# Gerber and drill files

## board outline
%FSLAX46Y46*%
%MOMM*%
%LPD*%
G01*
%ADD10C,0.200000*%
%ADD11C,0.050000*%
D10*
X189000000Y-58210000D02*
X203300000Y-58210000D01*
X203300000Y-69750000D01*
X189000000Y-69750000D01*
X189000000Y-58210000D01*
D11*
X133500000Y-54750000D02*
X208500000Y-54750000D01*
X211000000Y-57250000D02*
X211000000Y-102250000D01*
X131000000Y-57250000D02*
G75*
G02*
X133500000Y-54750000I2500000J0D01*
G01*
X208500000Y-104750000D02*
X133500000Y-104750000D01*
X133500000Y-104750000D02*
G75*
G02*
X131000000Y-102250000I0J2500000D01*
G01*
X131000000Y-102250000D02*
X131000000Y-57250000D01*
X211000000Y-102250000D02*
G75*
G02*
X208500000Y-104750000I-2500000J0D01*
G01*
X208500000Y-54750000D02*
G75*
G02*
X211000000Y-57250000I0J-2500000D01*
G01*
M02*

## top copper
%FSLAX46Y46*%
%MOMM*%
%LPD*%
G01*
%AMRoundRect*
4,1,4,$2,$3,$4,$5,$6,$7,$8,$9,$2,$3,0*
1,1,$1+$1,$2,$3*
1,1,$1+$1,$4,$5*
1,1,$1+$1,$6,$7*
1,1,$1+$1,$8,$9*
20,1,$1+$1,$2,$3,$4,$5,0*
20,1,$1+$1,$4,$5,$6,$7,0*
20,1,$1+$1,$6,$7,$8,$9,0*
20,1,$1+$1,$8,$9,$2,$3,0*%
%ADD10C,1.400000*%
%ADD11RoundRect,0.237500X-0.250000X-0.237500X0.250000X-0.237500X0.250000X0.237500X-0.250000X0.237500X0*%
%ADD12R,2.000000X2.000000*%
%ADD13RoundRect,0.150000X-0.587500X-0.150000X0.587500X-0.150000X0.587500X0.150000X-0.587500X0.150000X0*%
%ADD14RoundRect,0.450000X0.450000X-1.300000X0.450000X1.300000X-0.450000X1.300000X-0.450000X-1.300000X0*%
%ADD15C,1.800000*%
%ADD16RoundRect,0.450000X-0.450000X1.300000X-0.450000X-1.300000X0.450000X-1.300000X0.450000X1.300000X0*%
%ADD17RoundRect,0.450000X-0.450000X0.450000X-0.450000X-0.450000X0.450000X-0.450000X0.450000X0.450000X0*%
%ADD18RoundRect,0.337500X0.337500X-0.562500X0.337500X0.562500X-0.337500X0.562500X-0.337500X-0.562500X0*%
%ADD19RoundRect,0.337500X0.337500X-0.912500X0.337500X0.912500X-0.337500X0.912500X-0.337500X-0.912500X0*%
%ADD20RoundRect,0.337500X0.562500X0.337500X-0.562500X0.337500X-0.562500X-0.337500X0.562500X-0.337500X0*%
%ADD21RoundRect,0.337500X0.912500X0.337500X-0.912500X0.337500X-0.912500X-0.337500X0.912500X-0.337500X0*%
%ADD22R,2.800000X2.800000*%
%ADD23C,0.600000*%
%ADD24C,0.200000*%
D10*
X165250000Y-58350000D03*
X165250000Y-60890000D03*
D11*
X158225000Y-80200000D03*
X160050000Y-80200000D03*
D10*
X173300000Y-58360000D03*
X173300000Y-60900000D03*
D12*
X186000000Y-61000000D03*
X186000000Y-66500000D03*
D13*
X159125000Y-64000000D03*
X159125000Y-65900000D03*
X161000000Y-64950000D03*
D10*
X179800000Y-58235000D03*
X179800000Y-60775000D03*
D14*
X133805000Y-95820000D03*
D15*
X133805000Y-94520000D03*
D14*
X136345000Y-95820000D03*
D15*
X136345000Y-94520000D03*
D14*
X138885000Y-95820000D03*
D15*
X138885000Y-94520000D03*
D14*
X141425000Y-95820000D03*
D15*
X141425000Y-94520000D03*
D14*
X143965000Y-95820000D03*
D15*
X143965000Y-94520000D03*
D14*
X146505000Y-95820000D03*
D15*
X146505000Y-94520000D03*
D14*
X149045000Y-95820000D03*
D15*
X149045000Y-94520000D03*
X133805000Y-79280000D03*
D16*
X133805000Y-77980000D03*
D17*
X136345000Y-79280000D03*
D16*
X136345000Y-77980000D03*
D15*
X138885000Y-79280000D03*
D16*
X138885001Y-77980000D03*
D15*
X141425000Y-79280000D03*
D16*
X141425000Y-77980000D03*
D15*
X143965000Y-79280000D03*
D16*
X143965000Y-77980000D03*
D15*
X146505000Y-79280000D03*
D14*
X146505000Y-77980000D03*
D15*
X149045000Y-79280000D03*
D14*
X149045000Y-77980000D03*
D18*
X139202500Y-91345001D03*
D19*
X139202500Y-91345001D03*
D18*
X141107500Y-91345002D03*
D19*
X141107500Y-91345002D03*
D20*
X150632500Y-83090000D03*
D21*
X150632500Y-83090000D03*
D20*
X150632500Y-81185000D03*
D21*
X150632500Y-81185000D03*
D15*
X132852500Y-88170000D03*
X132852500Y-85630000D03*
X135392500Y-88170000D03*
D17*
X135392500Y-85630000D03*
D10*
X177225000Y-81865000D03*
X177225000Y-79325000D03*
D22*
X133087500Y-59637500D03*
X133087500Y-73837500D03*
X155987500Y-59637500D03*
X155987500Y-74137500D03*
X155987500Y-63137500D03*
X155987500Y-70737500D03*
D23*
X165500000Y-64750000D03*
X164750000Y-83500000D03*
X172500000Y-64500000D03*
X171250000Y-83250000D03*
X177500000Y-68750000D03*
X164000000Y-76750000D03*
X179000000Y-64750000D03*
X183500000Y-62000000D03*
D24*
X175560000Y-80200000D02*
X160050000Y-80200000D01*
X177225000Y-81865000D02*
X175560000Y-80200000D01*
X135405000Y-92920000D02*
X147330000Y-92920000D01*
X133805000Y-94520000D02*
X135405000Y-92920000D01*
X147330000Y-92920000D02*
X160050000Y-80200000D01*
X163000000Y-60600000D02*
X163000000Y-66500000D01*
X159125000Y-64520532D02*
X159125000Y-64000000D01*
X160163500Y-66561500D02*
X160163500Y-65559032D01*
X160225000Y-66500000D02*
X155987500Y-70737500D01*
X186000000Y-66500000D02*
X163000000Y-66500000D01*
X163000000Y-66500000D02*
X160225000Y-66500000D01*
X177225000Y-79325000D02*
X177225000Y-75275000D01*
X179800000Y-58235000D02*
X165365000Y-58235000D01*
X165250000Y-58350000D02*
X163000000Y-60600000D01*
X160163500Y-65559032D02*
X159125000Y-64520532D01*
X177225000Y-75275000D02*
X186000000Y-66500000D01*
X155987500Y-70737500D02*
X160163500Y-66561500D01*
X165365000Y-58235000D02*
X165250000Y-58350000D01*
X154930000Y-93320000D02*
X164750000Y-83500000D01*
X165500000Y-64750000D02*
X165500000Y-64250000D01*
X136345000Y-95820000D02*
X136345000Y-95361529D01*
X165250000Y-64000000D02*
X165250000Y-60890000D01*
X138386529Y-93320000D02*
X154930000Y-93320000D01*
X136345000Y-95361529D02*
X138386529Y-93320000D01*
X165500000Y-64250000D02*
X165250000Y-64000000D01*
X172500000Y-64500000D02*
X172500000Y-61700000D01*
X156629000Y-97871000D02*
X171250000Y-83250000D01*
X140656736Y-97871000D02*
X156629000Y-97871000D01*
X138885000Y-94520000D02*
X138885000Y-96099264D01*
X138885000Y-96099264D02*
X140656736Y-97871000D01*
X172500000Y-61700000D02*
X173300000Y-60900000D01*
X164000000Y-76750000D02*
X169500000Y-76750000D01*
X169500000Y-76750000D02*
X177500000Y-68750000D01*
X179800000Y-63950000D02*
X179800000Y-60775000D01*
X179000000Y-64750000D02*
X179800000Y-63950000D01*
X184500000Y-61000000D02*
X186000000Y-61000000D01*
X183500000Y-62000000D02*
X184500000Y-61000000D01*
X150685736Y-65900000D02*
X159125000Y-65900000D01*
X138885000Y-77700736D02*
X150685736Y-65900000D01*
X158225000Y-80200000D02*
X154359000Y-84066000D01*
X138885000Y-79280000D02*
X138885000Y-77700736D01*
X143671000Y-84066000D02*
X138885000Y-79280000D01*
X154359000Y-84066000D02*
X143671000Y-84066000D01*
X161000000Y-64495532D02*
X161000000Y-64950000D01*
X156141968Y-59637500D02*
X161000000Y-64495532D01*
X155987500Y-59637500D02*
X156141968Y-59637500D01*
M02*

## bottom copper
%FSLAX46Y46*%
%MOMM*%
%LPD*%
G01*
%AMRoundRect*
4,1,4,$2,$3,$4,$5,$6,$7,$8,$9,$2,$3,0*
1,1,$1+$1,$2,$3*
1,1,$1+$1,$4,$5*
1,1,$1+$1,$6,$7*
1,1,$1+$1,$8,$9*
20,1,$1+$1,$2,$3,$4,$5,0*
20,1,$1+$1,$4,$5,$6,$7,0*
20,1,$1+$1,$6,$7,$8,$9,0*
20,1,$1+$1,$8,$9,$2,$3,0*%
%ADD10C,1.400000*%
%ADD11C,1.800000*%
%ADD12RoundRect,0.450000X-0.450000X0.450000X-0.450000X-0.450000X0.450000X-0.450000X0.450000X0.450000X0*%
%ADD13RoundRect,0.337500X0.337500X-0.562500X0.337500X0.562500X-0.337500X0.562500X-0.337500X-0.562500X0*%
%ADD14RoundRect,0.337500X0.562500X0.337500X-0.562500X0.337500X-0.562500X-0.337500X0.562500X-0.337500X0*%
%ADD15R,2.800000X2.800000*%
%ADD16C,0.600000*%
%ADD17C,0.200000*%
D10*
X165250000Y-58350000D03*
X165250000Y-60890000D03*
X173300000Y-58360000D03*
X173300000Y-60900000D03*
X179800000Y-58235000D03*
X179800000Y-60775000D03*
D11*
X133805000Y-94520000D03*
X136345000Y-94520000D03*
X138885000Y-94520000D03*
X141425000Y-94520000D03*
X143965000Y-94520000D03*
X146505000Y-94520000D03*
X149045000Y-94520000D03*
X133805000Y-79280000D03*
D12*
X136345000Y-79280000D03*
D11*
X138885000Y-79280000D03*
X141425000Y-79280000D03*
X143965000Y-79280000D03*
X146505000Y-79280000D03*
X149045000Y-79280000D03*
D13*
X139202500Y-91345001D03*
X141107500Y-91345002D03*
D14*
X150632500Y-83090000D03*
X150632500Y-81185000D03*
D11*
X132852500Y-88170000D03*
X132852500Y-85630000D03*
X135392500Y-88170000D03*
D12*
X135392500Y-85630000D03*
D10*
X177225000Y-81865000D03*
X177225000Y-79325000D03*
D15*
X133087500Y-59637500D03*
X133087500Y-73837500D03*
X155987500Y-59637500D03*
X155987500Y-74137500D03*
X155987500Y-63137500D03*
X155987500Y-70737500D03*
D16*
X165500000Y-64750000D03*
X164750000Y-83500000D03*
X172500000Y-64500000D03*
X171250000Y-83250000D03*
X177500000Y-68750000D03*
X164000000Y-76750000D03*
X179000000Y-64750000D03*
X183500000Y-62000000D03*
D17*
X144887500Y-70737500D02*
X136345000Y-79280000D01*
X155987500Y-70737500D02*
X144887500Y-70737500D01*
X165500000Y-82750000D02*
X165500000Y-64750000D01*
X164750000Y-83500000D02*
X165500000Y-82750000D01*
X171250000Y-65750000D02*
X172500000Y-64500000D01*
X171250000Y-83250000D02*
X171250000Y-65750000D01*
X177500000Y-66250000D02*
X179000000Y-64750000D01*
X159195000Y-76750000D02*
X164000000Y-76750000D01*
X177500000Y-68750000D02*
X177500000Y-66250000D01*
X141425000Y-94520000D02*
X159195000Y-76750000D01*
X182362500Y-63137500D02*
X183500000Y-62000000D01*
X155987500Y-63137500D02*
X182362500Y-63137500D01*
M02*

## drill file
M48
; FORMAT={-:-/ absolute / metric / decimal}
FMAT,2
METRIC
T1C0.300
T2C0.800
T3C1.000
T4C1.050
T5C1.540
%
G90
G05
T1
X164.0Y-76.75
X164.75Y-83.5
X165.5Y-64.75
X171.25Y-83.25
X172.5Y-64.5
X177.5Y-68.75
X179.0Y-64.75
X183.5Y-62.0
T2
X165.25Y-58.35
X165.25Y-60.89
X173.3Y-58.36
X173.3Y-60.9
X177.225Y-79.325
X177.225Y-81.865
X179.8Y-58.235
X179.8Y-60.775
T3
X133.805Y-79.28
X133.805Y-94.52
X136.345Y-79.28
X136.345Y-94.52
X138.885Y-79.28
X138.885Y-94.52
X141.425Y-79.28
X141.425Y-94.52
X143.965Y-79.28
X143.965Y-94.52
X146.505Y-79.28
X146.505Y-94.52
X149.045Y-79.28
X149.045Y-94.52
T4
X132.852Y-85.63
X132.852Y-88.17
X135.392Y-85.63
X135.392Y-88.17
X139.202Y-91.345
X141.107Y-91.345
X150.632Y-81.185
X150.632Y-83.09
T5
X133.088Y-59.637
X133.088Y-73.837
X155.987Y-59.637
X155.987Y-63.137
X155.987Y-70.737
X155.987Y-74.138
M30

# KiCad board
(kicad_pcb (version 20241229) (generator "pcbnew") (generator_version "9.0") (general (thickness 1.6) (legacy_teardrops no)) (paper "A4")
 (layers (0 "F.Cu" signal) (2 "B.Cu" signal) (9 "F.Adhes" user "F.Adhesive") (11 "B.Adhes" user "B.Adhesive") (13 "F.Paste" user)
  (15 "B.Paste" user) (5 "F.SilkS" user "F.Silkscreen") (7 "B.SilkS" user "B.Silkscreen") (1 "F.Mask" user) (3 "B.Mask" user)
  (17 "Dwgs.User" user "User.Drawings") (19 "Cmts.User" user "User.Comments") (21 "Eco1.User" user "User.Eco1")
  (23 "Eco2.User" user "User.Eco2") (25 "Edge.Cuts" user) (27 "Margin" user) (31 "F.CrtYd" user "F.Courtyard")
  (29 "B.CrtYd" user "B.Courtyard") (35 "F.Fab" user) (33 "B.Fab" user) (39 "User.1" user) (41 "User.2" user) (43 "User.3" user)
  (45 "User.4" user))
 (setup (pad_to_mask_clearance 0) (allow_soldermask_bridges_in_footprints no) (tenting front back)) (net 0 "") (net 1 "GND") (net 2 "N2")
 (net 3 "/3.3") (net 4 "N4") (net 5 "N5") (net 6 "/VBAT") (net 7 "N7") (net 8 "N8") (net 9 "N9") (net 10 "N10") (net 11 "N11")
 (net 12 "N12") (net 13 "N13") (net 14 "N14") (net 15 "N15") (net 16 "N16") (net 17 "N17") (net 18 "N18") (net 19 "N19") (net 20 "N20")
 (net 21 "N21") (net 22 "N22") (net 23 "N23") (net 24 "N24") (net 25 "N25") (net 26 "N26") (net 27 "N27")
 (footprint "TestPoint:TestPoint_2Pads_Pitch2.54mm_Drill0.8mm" (layer "F.Cu") (at 165.25 58.35 -90)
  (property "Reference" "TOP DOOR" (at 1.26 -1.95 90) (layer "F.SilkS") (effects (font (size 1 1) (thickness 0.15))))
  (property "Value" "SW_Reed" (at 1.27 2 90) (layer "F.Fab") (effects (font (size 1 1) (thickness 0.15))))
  (pad "1" thru_hole circle (at 0 0 270) (size 1.4 1.4) (drill 0.8) (layers "*.Cu" "*.Mask") (remove_unused_layers no) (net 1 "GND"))
  (pad "2" thru_hole circle (at 2.54 0 270) (size 1.4 1.4) (drill 0.8) (layers "*.Cu" "*.Mask") (remove_unused_layers no) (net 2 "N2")))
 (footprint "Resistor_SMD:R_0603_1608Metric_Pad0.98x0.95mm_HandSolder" (layer "F.Cu") (at 159.1375 80.2)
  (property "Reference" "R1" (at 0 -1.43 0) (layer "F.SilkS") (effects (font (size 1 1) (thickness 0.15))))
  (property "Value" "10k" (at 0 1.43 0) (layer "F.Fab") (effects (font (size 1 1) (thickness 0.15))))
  (pad "1" smd roundrect (at -0.9125 0) (size 0.975 0.95) (layers "F.Cu" "F.Mask" "F.Paste") (roundrect_rratio 0.25) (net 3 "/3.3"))
  (pad "2" smd roundrect (at 0.9125 0) (size 0.975 0.95) (layers "F.Cu" "F.Mask" "F.Paste") (roundrect_rratio 0.25) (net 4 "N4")))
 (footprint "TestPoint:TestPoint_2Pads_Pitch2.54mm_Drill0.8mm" (layer "F.Cu") (at 173.3 58.36 -90)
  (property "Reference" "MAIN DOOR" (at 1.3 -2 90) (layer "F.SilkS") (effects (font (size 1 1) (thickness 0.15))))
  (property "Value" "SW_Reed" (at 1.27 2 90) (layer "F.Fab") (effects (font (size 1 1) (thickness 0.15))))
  (pad "1" thru_hole circle (at 0 0 270) (size 1.4 1.4) (drill 0.8) (layers "*.Cu" "*.Mask") (remove_unused_layers no) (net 1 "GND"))
  (pad "2" thru_hole circle (at 2.54 0 270) (size 1.4 1.4) (drill 0.8) (layers "*.Cu" "*.Mask") (remove_unused_layers no) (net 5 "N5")))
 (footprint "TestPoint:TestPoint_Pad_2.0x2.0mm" (layer "F.Cu") (at 186 61)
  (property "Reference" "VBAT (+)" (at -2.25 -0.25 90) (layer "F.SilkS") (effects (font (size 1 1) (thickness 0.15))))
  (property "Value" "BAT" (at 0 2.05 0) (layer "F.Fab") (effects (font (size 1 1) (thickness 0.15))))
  (pad "1" smd rect (at 0 0) (size 2 2) (layers "F.Cu" "F.Mask") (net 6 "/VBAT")))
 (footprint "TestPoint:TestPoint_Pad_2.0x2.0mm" (layer "F.Cu") (at 186 66.5)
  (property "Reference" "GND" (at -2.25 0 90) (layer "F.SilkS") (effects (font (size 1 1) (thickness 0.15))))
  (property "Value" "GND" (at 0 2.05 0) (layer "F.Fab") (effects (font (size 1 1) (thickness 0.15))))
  (pad "1" smd rect (at 0 0) (size 2 2) (layers "F.Cu" "F.Mask") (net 1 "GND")))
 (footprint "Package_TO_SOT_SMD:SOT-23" (layer "F.Cu") (at 160.0625 64.95)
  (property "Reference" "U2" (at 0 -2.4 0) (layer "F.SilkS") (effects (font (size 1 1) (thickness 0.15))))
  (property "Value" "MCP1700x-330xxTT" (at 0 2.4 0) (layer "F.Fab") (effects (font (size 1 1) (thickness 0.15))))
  (pad "1" smd roundrect (at -0.9375 -0.95) (size 1.475 0.6) (layers "F.Cu" "F.Mask" "F.Paste") (roundrect_rratio 0.25) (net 1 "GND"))
  (pad "2" smd roundrect (at -0.9375 0.95) (size 1.475 0.6) (layers "F.Cu" "F.Mask" "F.Paste") (roundrect_rratio 0.25) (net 3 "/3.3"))
  (pad "3" smd roundrect (at 0.9375 0) (size 1.475 0.6) (layers "F.Cu" "F.Mask" "F.Paste") (roundrect_rratio 0.25) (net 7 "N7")))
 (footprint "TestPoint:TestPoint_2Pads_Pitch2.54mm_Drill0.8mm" (layer "F.Cu") (at 179.8 58.235 -90)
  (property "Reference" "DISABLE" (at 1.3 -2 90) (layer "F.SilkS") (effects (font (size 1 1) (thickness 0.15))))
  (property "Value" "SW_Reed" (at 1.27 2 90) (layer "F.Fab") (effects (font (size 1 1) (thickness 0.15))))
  (pad "1" thru_hole circle (at 0 0 270) (size 1.4 1.4) (drill 0.8) (layers "*.Cu" "*.Mask") (remove_unused_layers no) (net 1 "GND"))
  (pad "2" thru_hole circle (at 2.54 0 270) (size 1.4 1.4) (drill 0.8) (layers "*.Cu" "*.Mask") (remove_unused_layers no) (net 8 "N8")))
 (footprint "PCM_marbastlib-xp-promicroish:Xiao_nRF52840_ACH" (layer "F.Cu") (at 141.425 86.9 90)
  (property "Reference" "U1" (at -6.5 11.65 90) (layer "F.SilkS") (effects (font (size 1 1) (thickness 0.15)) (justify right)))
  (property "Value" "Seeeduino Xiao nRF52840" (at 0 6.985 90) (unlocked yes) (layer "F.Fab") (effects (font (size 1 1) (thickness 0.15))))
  (pad "1" smd roundrect (at -8.92 -7.62 90) (size 3.5 1.8) (layers "F.Cu" "F.Mask") (roundrect_rratio 0.25) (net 4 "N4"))
  (pad "1" thru_hole circle (at -7.62 -7.62 90) (size 1.8 1.8) (drill 1) (layers "*.Cu" "*.Mask") (remove_unused_layers no) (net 4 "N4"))
  (pad "2" smd roundrect (at -8.92 -5.08 90) (size 3.5 1.8) (layers "F.Cu" "F.Mask") (roundrect_rratio 0.25) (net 2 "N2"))
  (pad "2" thru_hole circle (at -7.62 -5.08 90) (size 1.8 1.8) (drill 1) (layers "*.Cu" "*.Mask") (remove_unused_layers no) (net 2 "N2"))
  (pad "3" smd roundrect (at -8.92 -2.54 90) (size 3.5 1.8) (layers "F.Cu" "F.Mask") (roundrect_rratio 0.25) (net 5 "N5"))
  (pad "3" thru_hole circle (at -7.62 -2.54 90) (size 1.8 1.8) (drill 1) (layers "*.Cu" "*.Mask") (remove_unused_layers no) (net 5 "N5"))
  (pad "4" smd roundrect (at -8.92 0 90) (size 3.5 1.8) (layers "F.Cu" "F.Mask") (roundrect_rratio 0.25) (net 8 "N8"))
  (pad "4" thru_hole circle (at -7.62 0 90) (size 1.8 1.8) (drill 1) (layers "*.Cu" "*.Mask") (remove_unused_layers no) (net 8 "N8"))
  (pad "5" smd roundrect (at -8.92 2.54 90) (size 3.5 1.8) (layers "F.Cu" "F.Mask") (roundrect_rratio 0.25) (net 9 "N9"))
  (pad "5" thru_hole circle (at -7.62 2.54 90) (size 1.8 1.8) (drill 1) (layers "*.Cu" "*.Mask") (remove_unused_layers no) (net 9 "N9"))
  (pad "6" smd roundrect (at -8.92 5.08 90) (size 3.5 1.8) (layers "F.Cu" "F.Mask") (roundrect_rratio 0.25) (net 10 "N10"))
  (pad "6" thru_hole circle (at -7.62 5.08 90) (size 1.8 1.8) (drill 1) (layers "*.Cu" "*.Mask") (remove_unused_layers no) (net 10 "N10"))
  (pad "7" smd roundrect (at -8.92 7.62 90) (size 3.5 1.8) (layers "F.Cu" "F.Mask") (roundrect_rratio 0.25) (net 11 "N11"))
  (pad "7" thru_hole circle (at -7.62 7.62 90) (size 1.8 1.8) (drill 1) (layers "*.Cu" "*.Mask") (remove_unused_layers no) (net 11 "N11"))
  (pad "8" thru_hole circle (at 7.62 -7.62 270) (size 1.8 1.8) (drill 1) (layers "*.Cu" "*.Mask") (remove_unused_layers no) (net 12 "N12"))
  (pad "8" smd roundrect (at 8.92 -7.62 270) (size 3.5 1.8) (layers "F.Cu" "F.Mask") (roundrect_rratio 0.25) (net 12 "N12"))
  (pad "9" thru_hole roundrect (at 7.62 -5.08 270) (size 1.8 1.8) (drill 1) (layers "*.Cu" "*.Mask") (remove_unused_layers no)
   (roundrect_rratio 0.25) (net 1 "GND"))
  (pad "9" smd roundrect (at 8.92 -5.08 270) (size 3.5 1.8) (layers "F.Cu" "F.Mask") (roundrect_rratio 0.25) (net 1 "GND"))
  (pad "10" thru_hole circle (at 7.62 -2.54 270) (size 1.8 1.8) (drill 1) (layers "*.Cu" "*.Mask") (remove_unused_layers no) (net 3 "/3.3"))
  (pad "10" smd roundrect (at 8.92 -2.539999 270) (size 3.5 1.8) (layers "F.Cu" "F.Mask") (roundrect_rratio 0.25) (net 3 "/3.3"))
  (pad "11" thru_hole circle (at 7.62 0 270) (size 1.8 1.8) (drill 1) (layers "*.Cu" "*.Mask") (remove_unused_layers no) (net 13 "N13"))
  (pad "11" smd roundrect (at 8.92 0 270) (size 3.5 1.8) (layers "F.Cu" "F.Mask") (roundrect_rratio 0.25) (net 13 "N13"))
  (pad "12" thru_hole circle (at 7.62 2.54 270) (size 1.8 1.8) (drill 1) (layers "*.Cu" "*.Mask") (remove_unused_layers no) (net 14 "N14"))
  (pad "12" smd roundrect (at 8.92 2.54 270) (size 3.5 1.8) (layers "F.Cu" "F.Mask") (roundrect_rratio 0.25) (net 14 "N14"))
  (pad "13" thru_hole circle (at 7.62 5.08 90) (size 1.8 1.8) (drill 1) (layers "*.Cu" "*.Mask") (remove_unused_layers no) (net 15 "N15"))
  (pad "13" smd roundrect (at 8.92 5.08 90) (size 3.5 1.8) (layers "F.Cu" "F.Mask") (roundrect_rratio 0.25) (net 15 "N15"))
  (pad "14" thru_hole circle (at 7.62 7.62 90) (size 1.8 1.8) (drill 1) (layers "*.Cu" "*.Mask") (remove_unused_layers no) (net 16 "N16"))
  (pad "14" smd roundrect (at 8.92 7.62 90) (size 3.5 1.8) (layers "F.Cu" "F.Mask") (roundrect_rratio 0.25) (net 16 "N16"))
  (pad "15" thru_hole roundrect (at -4.445001 -2.2225 90) (size 1.8 1.35) (drill 1.05) (layers "*.Cu" "*.Mask") (remove_unused_layers no)
   (roundrect_rratio 0.25) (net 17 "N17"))
  (pad "15" smd roundrect (at -4.445001 -2.2225 90) (size 2.5 1.35) (layers "F.Cu" "F.Mask") (roundrect_rratio 0.25) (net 17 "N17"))
  (pad "16" thru_hole roundrect (at -4.445002 -0.3175 90) (size 1.8 1.35) (drill 1.05) (layers "*.Cu" "*.Mask") (remove_unused_layers no)
   (roundrect_rratio 0.25) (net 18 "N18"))
  (pad "16" smd roundrect (at -4.445002 -0.3175 90) (size 2.5 1.35) (layers "F.Cu" "F.Mask") (roundrect_rratio 0.25) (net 18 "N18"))
  (pad "17" thru_hole roundrect (at 3.81 9.2075 180) (size 1.8 1.35) (drill 1.05) (layers "*.Cu" "*.Mask") (remove_unused_layers no)
   (roundrect_rratio 0.25) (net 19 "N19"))
  (pad "17" smd roundrect (at 3.81 9.2075 180) (size 2.5 1.35) (layers "F.Cu" "F.Mask") (roundrect_rratio 0.25) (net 19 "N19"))
  (pad "18" thru_hole roundrect (at 5.715 9.2075 180) (size 1.8 1.35) (drill 1.05) (layers "*.Cu" "*.Mask") (remove_unused_layers no)
   (roundrect_rratio 0.25) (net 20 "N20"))
  (pad "18" smd roundrect (at 5.715 9.2075 180) (size 2.5 1.35) (layers "F.Cu" "F.Mask") (roundrect_rratio 0.25) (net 20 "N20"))
  (pad "19" thru_hole circle (at -1.27 -8.5725 270) (size 1.8 1.8) (drill 1.05) (layers "*.Cu" "*.Mask") (remove_unused_layers no)
   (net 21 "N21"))
  (pad "20" thru_hole circle (at 1.27 -8.5725 270) (size 1.8 1.8) (drill 1.05) (layers "*.Cu" "*.Mask") (remove_unused_layers no)
   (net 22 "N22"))
  (pad "21" thru_hole circle (at -1.27 -6.0325 270) (size 1.8 1.8) (drill 1.05) (layers "*.Cu" "*.Mask") (remove_unused_layers no)
   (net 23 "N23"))
  (pad "22" thru_hole roundrect (at 1.27 -6.0325 270) (size 1.8 1.8) (drill 1.05) (layers "*.Cu" "*.Mask") (remove_unused_layers no)
   (roundrect_rratio 0.25) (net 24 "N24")))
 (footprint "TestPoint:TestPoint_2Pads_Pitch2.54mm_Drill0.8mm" (layer "F.Cu") (at 177.225 81.865 90)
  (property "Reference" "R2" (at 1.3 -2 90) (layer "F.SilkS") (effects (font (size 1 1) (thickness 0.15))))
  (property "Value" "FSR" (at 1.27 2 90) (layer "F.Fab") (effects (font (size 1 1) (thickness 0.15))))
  (pad "1" thru_hole circle (at 0 0 90) (size 1.4 1.4) (drill 0.8) (layers "*.Cu" "*.Mask") (remove_unused_layers no) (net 4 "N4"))
  (pad "2" thru_hole circle (at 2.54 0 90) (size 1.4 1.4) (drill 0.8) (layers "*.Cu" "*.Mask") (remove_unused_layers no) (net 1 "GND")))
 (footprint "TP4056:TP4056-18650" (layer "F.Cu") (at 131.3875 57.9375)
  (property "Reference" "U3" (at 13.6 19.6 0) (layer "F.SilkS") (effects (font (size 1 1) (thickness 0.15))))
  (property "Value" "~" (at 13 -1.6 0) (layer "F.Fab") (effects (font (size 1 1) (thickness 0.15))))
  (pad "1" thru_hole rect (at 1.7 1.7) (size 2.8 2.8) (drill 1.54) (layers "*.Cu" "*.Mask") (remove_unused_layers no) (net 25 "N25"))
  (pad "2" thru_hole rect (at 1.7 15.9) (size 2.8 2.8) (drill 1.54) (layers "*.Cu" "*.Mask") (remove_unused_layers no) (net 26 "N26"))
  (pad "3" thru_hole rect (at 24.6 1.7) (size 2.8 2.8) (drill 1.54) (layers "*.Cu" "*.Mask") (remove_unused_layers no) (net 7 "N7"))
  (pad "4" thru_hole rect (at 24.6 16.2) (size 2.8 2.8) (drill 1.54) (layers "*.Cu" "*.Mask") (remove_unused_layers no) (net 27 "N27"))
  (pad "5" thru_hole rect (at 24.6 5.2) (size 2.8 2.8) (drill 1.54) (layers "*.Cu" "*.Mask") (remove_unused_layers no) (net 6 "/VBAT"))
  (pad "6" thru_hole rect (at 24.6 12.8) (size 2.8 2.8) (drill 1.54) (layers "*.Cu" "*.Mask") (remove_unused_layers no) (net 1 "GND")))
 (gr_rect (start 189 58.21) (end 203.3 69.75) (stroke (width 0.2) (type default)) (fill no) (layer "Edge.Cuts"))
 (gr_line (start 133.5 54.75) (end 208.5 54.75) (stroke (width 0.05) (type default)) (layer "Edge.Cuts"))
 (gr_line (start 211 57.25) (end 211 102.25) (stroke (width 0.05) (type default)) (layer "Edge.Cuts"))
 (gr_arc (start 131 57.25) (mid 131.732233 55.482233) (end 133.5 54.75) (stroke (width 0.05) (type default)) (layer "Edge.Cuts"))
 (gr_line (start 208.5 104.75) (end 133.5 104.75) (stroke (width 0.05) (type default)) (layer "Edge.Cuts"))
 (gr_arc (start 133.5 104.75) (mid 131.732233 104.017767) (end 131 102.25) (stroke (width 0.05) (type default)) (layer "Edge.Cuts"))
 (gr_line (start 131 102.25) (end 131 57.25) (stroke (width 0.05) (type default)) (layer "Edge.Cuts"))
 (gr_arc (start 211 102.25) (mid 210.267767 104.017767) (end 208.5 104.75) (stroke (width 0.05) (type default)) (layer "Edge.Cuts"))
 (gr_arc (start 208.5 54.75) (mid 210.267767 55.482233) (end 211 57.25) (stroke (width 0.05) (type default)) (layer "Edge.Cuts"))
 (segment (start 175.56 80.2) (end 160.05 80.2) (width 0.2) (layer "F.Cu") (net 4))
 (segment (start 177.225 81.865) (end 175.56 80.2) (width 0.2) (layer "F.Cu") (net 4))
 (segment (start 135.405 92.92) (end 147.33 92.92) (width 0.2) (layer "F.Cu") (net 4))
 (segment (start 133.805 94.52) (end 135.405 92.92) (width 0.2) (layer "F.Cu") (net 4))
 (segment (start 147.33 92.92) (end 160.05 80.2) (width 0.2) (layer "F.Cu") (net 4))
 (segment (start 163 60.6) (end 163 66.5) (width 0.2) (layer "F.Cu") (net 1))
 (segment (start 159.125 64.520532) (end 159.125 64) (width 0.2) (layer "F.Cu") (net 1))
 (segment (start 160.1635 66.5615) (end 160.1635 65.559032) (width 0.2) (layer "F.Cu") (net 1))
 (segment (start 160.225 66.5) (end 155.9875 70.7375) (width 0.2) (layer "F.Cu") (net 1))
 (segment (start 186 66.5) (end 163 66.5) (width 0.2) (layer "F.Cu") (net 1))
 (segment (start 163 66.5) (end 160.225 66.5) (width 0.2) (layer "F.Cu") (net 1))
 (segment (start 177.225 79.325) (end 177.225 75.275) (width 0.2) (layer "F.Cu") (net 1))
 (segment (start 179.8 58.235) (end 165.365 58.235) (width 0.2) (layer "F.Cu") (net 1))
 (segment (start 165.25 58.35) (end 163 60.6) (width 0.2) (layer "F.Cu") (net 1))
 (segment (start 160.1635 65.559032) (end 159.125 64.520532) (width 0.2) (layer "F.Cu") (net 1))
 (segment (start 177.225 75.275) (end 186 66.5) (width 0.2) (layer "F.Cu") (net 1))
 (segment (start 155.9875 70.7375) (end 160.1635 66.5615) (width 0.2) (layer "F.Cu") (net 1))
 (segment (start 165.365 58.235) (end 165.25 58.35) (width 0.2) (layer "F.Cu") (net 1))
 (segment (start 144.8875 70.7375) (end 136.345 79.28) (width 0.2) (layer "B.Cu") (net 1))
 (segment (start 155.9875 70.7375) (end 144.8875 70.7375) (width 0.2) (layer "B.Cu") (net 1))
 (segment (start 154.93 93.32) (end 164.75 83.5) (width 0.2) (layer "F.Cu") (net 2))
 (segment (start 165.5 64.75) (end 165.5 64.25) (width 0.2) (layer "F.Cu") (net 2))
 (segment (start 136.345 95.82) (end 136.345 95.361529) (width 0.2) (layer "F.Cu") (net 2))
 (segment (start 165.25 64) (end 165.25 60.89) (width 0.2) (layer "F.Cu") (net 2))
 (segment (start 138.386529 93.32) (end 154.93 93.32) (width 0.2) (layer "F.Cu") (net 2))
 (segment (start 136.345 95.361529) (end 138.386529 93.32) (width 0.2) (layer "F.Cu") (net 2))
 (segment (start 165.5 64.25) (end 165.25 64) (width 0.2) (layer "F.Cu") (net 2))
 (via (at 165.5 64.75) (size 0.6) (drill 0.3) (layers "F.Cu" "B.Cu") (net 2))
 (via (at 164.75 83.5) (size 0.6) (drill 0.3) (layers "F.Cu" "B.Cu") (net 2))
 (segment (start 165.5 82.75) (end 165.5 64.75) (width 0.2) (layer "B.Cu") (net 2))
 (segment (start 164.75 83.5) (end 165.5 82.75) (width 0.2) (layer "B.Cu") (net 2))
 (segment (start 172.5 64.5) (end 172.5 61.7) (width 0.2) (layer "F.Cu") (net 5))
 (segment (start 156.629 97.871) (end 171.25 83.25) (width 0.2) (layer "F.Cu") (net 5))
 (segment (start 140.656736 97.871) (end 156.629 97.871) (width 0.2) (layer "F.Cu") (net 5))
 (segment (start 138.885 94.52) (end 138.885 96.099264) (width 0.2) (layer "F.Cu") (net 5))
 (segment (start 138.885 96.099264) (end 140.656736 97.871) (width 0.2) (layer "F.Cu") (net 5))
 (segment (start 172.5 61.7) (end 173.3 60.9) (width 0.2) (layer "F.Cu") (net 5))
 (via (at 172.5 64.5) (size 0.6) (drill 0.3) (layers "F.Cu" "B.Cu") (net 5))
 (via (at 171.25 83.25) (size 0.6) (drill 0.3) (layers "F.Cu" "B.Cu") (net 5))
 (segment (start 171.25 65.75) (end 172.5 64.5) (width 0.2) (layer "B.Cu") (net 5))
 (segment (start 171.25 83.25) (end 171.25 65.75) (width 0.2) (layer "B.Cu") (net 5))
 (segment (start 164 76.75) (end 169.5 76.75) (width 0.2) (layer "F.Cu") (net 8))
 (segment (start 169.5 76.75) (end 177.5 68.75) (width 0.2) (layer "F.Cu") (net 8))
 (segment (start 179.8 63.95) (end 179.8 60.775) (width 0.2) (layer "F.Cu") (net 8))
 (segment (start 179 64.75) (end 179.8 63.95) (width 0.2) (layer "F.Cu") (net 8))
 (via (at 177.5 68.75) (size 0.6) (drill 0.3) (layers "F.Cu" "B.Cu") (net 8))
 (via (at 164 76.75) (size 0.6) (drill 0.3) (layers "F.Cu" "B.Cu") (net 8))
 (via (at 179 64.75) (size 0.6) (drill 0.3) (layers "F.Cu" "B.Cu") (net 8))
 (segment (start 177.5 66.25) (end 179 64.75) (width 0.2) (layer "B.Cu") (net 8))
 (segment (start 159.195 76.75) (end 164 76.75) (width 0.2) (layer "B.Cu") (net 8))
 (segment (start 177.5 68.75) (end 177.5 66.25) (width 0.2) (layer "B.Cu") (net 8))
 (segment (start 141.425 94.52) (end 159.195 76.75) (width 0.2) (layer "B.Cu") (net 8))
 (segment (start 184.5 61) (end 186 61) (width 0.2) (layer "F.Cu") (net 6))
 (segment (start 183.5 62) (end 184.5 61) (width 0.2) (layer "F.Cu") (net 6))
 (via (at 183.5 62) (size 0.6) (drill 0.3) (layers "F.Cu" "B.Cu") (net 6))
 (segment (start 182.3625 63.1375) (end 183.5 62) (width 0.2) (layer "B.Cu") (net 6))
 (segment (start 155.9875 63.1375) (end 182.3625 63.1375) (width 0.2) (layer "B.Cu") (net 6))
 (segment (start 150.685736 65.9) (end 159.125 65.9) (width 0.2) (layer "F.Cu") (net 3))
 (segment (start 138.885 77.700736) (end 150.685736 65.9) (width 0.2) (layer "F.Cu") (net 3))
 (segment (start 158.225 80.2) (end 154.359 84.066) (width 0.2) (layer "F.Cu") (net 3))
 (segment (start 138.885 79.28) (end 138.885 77.700736) (width 0.2) (layer "F.Cu") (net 3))
 (segment (start 143.671 84.066) (end 138.885 79.28) (width 0.2) (layer "F.Cu") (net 3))
 (segment (start 154.359 84.066) (end 143.671 84.066) (width 0.2) (layer "F.Cu") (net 3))
 (segment (start 161 64.495532) (end 161 64.95) (width 0.2) (layer "F.Cu") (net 7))
 (segment (start 156.141968 59.6375) (end 161 64.495532) (width 0.2) (layer "F.Cu") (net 7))
 (segment (start 155.9875 59.6375) (end 156.141968 59.6375) (width 0.2) (layer "F.Cu") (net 7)))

